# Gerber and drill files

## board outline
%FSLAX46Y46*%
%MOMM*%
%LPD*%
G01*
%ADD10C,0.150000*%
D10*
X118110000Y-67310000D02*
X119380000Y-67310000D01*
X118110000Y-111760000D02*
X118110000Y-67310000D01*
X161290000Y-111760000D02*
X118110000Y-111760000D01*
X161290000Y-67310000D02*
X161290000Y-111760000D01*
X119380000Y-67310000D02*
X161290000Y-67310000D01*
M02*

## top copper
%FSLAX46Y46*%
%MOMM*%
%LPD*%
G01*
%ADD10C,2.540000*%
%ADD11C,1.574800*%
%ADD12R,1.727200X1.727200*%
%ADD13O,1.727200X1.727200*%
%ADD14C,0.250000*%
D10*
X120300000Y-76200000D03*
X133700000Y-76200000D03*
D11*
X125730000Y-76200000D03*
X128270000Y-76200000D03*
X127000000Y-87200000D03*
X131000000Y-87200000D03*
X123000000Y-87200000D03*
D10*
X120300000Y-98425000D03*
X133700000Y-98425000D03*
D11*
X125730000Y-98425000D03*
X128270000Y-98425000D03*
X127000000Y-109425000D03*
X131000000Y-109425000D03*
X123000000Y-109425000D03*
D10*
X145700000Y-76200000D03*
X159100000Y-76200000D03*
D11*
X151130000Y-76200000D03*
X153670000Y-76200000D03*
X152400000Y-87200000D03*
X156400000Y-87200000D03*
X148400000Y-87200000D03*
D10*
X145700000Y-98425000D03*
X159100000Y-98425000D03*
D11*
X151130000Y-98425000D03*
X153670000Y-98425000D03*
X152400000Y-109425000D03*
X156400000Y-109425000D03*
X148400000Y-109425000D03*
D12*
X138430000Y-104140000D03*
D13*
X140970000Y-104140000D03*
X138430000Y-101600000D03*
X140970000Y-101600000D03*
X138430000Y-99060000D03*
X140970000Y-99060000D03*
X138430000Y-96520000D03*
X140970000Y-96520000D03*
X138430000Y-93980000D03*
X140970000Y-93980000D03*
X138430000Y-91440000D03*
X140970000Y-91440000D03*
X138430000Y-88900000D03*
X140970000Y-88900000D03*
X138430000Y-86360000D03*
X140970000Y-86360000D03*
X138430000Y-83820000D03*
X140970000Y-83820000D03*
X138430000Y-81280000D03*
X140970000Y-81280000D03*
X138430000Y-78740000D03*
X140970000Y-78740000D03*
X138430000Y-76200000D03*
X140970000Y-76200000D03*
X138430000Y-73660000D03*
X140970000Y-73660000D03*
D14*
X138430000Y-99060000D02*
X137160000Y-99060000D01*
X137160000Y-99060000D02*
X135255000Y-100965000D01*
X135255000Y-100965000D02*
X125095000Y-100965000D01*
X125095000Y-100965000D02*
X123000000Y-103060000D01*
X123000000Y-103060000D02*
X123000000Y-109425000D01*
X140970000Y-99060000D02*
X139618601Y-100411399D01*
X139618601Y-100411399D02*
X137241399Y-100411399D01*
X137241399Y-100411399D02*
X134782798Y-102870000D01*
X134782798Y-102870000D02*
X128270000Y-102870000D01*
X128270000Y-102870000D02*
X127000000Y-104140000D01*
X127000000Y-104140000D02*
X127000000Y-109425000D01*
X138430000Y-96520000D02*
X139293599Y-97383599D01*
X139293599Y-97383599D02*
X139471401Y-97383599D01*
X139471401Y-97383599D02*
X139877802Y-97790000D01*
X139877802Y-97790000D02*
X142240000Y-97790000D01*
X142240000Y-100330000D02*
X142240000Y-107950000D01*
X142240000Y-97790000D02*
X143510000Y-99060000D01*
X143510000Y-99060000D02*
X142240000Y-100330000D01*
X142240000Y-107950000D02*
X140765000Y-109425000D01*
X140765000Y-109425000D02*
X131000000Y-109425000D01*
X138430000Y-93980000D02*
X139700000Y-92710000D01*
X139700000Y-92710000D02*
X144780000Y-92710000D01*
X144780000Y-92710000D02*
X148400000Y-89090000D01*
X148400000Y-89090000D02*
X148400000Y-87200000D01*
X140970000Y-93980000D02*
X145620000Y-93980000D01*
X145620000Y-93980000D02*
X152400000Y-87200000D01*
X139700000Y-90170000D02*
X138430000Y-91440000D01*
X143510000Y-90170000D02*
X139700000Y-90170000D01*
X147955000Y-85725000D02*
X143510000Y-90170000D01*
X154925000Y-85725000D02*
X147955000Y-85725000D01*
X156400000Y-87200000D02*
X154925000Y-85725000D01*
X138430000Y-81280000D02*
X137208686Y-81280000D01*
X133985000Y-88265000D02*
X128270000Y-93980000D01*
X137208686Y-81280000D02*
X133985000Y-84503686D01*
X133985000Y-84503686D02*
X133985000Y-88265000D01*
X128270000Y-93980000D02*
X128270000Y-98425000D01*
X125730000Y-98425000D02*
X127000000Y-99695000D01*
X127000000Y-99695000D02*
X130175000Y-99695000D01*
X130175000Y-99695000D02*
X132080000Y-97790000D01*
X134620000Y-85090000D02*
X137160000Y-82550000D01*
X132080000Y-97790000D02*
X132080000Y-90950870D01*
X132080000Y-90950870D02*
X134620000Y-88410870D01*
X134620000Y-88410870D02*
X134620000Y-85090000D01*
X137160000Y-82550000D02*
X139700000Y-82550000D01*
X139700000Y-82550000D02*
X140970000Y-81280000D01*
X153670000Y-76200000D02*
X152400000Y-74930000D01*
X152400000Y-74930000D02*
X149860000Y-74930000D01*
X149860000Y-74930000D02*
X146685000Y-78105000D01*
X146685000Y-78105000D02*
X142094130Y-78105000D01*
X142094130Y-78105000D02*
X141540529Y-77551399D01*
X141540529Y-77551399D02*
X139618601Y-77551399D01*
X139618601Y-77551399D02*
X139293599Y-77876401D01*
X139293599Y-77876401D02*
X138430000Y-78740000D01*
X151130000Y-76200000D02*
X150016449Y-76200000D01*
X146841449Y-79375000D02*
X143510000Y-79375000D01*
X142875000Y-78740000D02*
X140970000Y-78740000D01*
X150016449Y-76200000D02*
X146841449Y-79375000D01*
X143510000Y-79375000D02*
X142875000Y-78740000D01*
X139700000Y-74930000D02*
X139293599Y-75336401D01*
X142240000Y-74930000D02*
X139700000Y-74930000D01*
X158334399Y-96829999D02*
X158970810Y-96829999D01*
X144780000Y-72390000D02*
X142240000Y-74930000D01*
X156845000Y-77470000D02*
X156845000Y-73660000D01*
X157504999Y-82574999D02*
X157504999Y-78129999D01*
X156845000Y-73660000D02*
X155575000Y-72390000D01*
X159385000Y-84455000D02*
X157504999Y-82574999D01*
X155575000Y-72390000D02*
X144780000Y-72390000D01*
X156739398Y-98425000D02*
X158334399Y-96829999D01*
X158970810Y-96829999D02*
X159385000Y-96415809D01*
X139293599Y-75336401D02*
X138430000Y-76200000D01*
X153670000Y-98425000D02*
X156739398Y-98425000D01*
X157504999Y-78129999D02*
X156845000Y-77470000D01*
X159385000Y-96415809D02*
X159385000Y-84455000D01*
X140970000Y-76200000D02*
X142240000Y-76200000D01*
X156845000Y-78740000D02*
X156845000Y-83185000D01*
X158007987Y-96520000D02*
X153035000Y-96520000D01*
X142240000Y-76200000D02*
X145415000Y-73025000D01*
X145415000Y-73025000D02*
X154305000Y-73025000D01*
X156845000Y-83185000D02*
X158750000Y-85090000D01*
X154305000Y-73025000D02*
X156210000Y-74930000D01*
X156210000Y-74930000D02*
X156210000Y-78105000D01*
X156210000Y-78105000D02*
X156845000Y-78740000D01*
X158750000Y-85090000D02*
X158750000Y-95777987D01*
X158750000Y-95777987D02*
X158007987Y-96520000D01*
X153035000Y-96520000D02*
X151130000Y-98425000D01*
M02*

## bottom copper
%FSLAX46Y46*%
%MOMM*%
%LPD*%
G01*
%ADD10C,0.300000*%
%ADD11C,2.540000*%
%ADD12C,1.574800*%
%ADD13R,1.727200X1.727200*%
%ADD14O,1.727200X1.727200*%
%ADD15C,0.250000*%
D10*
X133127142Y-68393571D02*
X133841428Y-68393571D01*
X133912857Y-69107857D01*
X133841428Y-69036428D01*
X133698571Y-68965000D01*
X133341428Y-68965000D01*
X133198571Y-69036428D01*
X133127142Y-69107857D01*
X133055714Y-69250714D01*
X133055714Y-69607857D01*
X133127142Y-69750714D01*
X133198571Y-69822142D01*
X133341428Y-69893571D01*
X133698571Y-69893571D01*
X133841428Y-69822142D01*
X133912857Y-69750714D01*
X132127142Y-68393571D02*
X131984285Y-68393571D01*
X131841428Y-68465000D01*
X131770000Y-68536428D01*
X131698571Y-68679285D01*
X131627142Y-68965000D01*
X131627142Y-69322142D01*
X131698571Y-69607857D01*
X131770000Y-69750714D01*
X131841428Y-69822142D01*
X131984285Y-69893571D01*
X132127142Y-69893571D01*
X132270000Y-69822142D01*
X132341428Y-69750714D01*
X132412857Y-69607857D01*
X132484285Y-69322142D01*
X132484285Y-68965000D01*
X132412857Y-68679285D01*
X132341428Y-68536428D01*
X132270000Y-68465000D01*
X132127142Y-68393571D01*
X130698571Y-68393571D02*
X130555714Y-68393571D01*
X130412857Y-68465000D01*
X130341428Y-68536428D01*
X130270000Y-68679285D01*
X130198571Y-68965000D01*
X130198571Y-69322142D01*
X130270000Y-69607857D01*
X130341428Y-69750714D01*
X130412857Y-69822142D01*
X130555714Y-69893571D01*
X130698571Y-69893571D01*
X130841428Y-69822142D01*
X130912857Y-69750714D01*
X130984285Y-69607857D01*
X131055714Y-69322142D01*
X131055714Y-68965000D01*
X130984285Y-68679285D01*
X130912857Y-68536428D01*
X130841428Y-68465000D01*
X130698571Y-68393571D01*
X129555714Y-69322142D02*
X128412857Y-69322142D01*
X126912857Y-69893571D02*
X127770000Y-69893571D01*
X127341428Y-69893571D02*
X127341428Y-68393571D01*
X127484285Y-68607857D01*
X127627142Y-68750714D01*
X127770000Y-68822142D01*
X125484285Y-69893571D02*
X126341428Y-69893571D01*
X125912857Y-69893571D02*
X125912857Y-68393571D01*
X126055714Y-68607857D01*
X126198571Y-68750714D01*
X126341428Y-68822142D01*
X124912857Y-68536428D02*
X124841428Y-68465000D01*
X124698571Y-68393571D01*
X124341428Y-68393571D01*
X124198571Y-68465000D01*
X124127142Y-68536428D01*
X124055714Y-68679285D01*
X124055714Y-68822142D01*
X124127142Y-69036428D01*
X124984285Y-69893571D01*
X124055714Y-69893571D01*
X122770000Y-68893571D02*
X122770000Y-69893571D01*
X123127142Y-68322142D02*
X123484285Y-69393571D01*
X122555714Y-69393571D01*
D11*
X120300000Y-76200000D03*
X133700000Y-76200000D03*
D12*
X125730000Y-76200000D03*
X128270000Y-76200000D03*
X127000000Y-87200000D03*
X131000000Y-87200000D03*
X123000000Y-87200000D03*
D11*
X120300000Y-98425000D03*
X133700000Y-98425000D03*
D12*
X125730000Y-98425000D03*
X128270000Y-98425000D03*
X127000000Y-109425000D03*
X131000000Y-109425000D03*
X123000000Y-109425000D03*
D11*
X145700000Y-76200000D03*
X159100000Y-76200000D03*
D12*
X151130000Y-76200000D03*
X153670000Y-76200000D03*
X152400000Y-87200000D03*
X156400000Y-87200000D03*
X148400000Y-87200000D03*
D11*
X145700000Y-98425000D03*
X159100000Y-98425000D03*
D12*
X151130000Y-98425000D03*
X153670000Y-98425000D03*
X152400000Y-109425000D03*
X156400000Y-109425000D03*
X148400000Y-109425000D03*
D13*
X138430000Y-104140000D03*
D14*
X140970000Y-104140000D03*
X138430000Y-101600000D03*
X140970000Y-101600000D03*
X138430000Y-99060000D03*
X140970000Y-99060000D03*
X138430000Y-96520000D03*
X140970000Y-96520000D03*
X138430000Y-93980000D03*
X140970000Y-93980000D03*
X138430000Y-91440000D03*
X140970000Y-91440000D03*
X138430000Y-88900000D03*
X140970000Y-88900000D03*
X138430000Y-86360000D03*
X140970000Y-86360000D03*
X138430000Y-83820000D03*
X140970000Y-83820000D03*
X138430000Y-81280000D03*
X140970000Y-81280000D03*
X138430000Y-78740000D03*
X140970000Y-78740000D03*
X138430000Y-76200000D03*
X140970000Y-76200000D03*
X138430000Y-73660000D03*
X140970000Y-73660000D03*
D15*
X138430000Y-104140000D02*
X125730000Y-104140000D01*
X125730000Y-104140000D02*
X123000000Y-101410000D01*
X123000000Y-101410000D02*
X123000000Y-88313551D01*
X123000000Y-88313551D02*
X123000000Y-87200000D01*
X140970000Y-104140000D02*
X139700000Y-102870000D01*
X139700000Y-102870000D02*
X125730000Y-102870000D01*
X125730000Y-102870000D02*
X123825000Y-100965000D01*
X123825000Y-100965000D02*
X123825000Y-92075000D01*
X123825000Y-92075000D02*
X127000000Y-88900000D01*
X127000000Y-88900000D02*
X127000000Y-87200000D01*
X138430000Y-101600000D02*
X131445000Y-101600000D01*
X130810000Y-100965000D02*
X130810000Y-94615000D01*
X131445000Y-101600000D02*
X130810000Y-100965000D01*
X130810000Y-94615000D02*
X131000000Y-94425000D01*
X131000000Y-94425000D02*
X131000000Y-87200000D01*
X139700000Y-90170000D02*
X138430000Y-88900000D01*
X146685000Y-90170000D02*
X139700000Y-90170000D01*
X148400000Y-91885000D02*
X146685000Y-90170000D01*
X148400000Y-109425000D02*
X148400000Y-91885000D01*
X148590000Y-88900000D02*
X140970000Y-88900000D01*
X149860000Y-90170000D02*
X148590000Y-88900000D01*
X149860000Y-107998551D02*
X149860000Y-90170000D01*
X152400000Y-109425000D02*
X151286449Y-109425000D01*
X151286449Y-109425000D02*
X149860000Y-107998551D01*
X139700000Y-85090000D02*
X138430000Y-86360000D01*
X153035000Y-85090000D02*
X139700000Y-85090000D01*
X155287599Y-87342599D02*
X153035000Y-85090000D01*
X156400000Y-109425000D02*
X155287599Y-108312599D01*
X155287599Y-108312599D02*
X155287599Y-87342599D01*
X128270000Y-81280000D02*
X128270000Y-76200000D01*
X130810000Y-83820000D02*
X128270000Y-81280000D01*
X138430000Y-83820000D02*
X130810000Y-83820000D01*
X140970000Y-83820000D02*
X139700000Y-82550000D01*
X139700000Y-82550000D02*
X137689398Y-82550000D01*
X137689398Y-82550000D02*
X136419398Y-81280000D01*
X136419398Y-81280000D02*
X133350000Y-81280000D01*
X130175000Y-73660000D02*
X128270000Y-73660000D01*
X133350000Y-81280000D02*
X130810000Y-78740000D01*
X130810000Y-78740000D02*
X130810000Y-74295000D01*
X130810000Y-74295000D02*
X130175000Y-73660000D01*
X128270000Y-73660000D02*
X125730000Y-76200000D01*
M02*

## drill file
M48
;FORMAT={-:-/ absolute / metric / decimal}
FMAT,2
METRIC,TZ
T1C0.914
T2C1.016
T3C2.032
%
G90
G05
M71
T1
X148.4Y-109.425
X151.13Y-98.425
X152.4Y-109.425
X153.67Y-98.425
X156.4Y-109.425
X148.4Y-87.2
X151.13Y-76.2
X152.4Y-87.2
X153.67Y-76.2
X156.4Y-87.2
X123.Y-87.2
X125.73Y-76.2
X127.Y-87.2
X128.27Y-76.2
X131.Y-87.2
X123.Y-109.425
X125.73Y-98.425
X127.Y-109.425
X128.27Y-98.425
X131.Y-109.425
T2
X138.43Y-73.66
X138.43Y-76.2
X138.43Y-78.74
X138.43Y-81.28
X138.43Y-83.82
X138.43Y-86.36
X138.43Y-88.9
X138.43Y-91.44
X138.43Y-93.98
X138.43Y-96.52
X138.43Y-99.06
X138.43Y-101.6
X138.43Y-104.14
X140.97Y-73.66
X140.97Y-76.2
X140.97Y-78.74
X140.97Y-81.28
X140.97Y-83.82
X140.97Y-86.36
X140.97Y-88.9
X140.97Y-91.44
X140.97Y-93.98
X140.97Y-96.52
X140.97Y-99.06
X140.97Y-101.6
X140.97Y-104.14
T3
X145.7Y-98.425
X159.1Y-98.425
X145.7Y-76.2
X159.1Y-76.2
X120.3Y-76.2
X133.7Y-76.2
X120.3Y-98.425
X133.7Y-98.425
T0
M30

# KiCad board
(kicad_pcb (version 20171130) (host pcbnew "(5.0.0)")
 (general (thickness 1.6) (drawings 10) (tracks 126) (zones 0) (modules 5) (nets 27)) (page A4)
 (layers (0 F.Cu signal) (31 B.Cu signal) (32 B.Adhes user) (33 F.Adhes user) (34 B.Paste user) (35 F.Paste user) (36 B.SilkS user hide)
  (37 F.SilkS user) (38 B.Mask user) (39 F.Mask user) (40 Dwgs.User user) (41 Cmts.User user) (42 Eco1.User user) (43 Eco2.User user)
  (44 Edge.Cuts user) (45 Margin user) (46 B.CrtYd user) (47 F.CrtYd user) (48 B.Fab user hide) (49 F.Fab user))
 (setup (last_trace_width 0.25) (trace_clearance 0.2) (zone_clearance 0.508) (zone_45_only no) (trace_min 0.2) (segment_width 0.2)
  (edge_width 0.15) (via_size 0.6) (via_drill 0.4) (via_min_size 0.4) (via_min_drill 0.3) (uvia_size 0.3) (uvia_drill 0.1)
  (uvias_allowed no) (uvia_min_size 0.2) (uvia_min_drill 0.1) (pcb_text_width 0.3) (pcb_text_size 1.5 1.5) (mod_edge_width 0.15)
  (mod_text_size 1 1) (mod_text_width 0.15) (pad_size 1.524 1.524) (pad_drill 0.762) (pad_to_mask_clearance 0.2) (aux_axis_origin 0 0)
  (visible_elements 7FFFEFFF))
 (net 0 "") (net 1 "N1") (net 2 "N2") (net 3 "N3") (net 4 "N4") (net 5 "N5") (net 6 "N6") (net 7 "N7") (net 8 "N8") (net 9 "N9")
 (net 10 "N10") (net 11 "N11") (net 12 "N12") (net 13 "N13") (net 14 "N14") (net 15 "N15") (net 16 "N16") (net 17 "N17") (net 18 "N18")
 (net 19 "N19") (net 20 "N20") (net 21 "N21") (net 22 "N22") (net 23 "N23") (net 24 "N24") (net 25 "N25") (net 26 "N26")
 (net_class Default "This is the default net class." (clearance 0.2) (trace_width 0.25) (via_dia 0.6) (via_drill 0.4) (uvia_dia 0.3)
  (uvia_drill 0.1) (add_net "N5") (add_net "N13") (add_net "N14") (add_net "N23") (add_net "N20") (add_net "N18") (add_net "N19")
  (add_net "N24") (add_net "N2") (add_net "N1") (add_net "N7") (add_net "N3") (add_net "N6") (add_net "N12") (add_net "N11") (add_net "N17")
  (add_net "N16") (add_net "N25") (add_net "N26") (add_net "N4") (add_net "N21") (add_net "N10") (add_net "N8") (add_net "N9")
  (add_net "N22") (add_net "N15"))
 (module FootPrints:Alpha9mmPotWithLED (layer F.Cu) (at 127 76.2)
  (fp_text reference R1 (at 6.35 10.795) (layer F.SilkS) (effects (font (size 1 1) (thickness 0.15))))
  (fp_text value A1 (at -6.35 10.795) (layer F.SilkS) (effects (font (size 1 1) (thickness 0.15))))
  (pad "" thru_hole circle (at -6.7 0) (size 2.54 2.54) (drill 2.032) (layers *.Cu *.Mask F.SilkS))
  (pad "" thru_hole circle (at 6.7 0) (size 2.54 2.54) (drill 2.032) (layers *.Cu *.Mask F.SilkS))
  (pad 4 thru_hole circle (at -1.27 0) (size 1.5748 1.5748) (drill 0.9144) (layers *.Cu *.Mask F.SilkS) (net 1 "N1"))
  (pad 5 thru_hole circle (at 1.27 0) (size 1.5748 1.5748) (drill 0.9144) (layers *.Cu *.Mask F.SilkS) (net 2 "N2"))
  (pad 2 thru_hole circle (at 0 11) (size 1.5748 1.5748) (drill 0.9144) (layers *.Cu *.Mask F.SilkS) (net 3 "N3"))
  (pad 3 thru_hole circle (at 4 11) (size 1.5748 1.5748) (drill 0.9144) (layers *.Cu *.Mask F.SilkS) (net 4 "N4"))
  (pad 1 thru_hole circle (at -4 11) (size 1.5748 1.5748) (drill 0.9144) (layers *.Cu *.Mask F.SilkS) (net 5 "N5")))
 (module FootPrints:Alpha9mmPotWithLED (layer F.Cu) (at 127 98.425)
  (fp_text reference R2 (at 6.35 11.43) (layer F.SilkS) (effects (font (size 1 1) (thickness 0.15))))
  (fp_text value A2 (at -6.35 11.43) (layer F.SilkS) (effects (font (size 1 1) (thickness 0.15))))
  (pad "" thru_hole circle (at -6.7 0) (size 2.54 2.54) (drill 2.032) (layers *.Cu *.Mask F.SilkS))
  (pad "" thru_hole circle (at 6.7 0) (size 2.54 2.54) (drill 2.032) (layers *.Cu *.Mask F.SilkS))
  (pad 4 thru_hole circle (at -1.27 0) (size 1.5748 1.5748) (drill 0.9144) (layers *.Cu *.Mask F.SilkS) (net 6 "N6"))
  (pad 5 thru_hole circle (at 1.27 0) (size 1.5748 1.5748) (drill 0.9144) (layers *.Cu *.Mask F.SilkS) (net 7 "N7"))
  (pad 2 thru_hole circle (at 0 11) (size 1.5748 1.5748) (drill 0.9144) (layers *.Cu *.Mask F.SilkS) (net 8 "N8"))
  (pad 3 thru_hole circle (at 4 11) (size 1.5748 1.5748) (drill 0.9144) (layers *.Cu *.Mask F.SilkS) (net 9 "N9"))
  (pad 1 thru_hole circle (at -4 11) (size 1.5748 1.5748) (drill 0.9144) (layers *.Cu *.Mask F.SilkS) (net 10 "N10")))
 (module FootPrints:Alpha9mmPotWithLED (layer F.Cu) (at 152.4 76.2)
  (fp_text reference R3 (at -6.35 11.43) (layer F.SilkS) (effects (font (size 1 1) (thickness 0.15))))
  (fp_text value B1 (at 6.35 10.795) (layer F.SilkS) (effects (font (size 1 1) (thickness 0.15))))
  (pad "" thru_hole circle (at -6.7 0) (size 2.54 2.54) (drill 2.032) (layers *.Cu *.Mask F.SilkS))
  (pad "" thru_hole circle (at 6.7 0) (size 2.54 2.54) (drill 2.032) (layers *.Cu *.Mask F.SilkS))
  (pad 4 thru_hole circle (at -1.27 0) (size 1.5748 1.5748) (drill 0.9144) (layers *.Cu *.Mask F.SilkS) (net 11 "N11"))
  (pad 5 thru_hole circle (at 1.27 0) (size 1.5748 1.5748) (drill 0.9144) (layers *.Cu *.Mask F.SilkS) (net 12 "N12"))
  (pad 2 thru_hole circle (at 0 11) (size 1.5748 1.5748) (drill 0.9144) (layers *.Cu *.Mask F.SilkS) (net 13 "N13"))
  (pad 3 thru_hole circle (at 4 11) (size 1.5748 1.5748) (drill 0.9144) (layers *.Cu *.Mask F.SilkS) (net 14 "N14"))
  (pad 1 thru_hole circle (at -4 11) (size 1.5748 1.5748) (drill 0.9144) (layers *.Cu *.Mask F.SilkS) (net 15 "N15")))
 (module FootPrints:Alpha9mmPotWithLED (layer F.Cu) (at 152.4 98.425)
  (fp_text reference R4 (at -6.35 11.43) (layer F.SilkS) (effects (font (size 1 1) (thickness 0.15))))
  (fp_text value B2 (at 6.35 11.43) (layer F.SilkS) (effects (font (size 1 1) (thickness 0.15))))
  (pad "" thru_hole circle (at -6.7 0) (size 2.54 2.54) (drill 2.032) (layers *.Cu *.Mask F.SilkS))
  (pad "" thru_hole circle (at 6.7 0) (size 2.54 2.54) (drill 2.032) (layers *.Cu *.Mask F.SilkS))
  (pad 4 thru_hole circle (at -1.27 0) (size 1.5748 1.5748) (drill 0.9144) (layers *.Cu *.Mask F.SilkS) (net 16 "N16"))
  (pad 5 thru_hole circle (at 1.27 0) (size 1.5748 1.5748) (drill 0.9144) (layers *.Cu *.Mask F.SilkS) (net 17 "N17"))
  (pad 2 thru_hole circle (at 0 11) (size 1.5748 1.5748) (drill 0.9144) (layers *.Cu *.Mask F.SilkS) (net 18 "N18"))
  (pad 3 thru_hole circle (at 4 11) (size 1.5748 1.5748) (drill 0.9144) (layers *.Cu *.Mask F.SilkS) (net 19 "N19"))
  (pad 1 thru_hole circle (at -4 11) (size 1.5748 1.5748) (drill 0.9144) (layers *.Cu *.Mask F.SilkS) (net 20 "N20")))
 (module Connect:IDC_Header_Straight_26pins (layer B.Cu) (at 138.43 104.14 90)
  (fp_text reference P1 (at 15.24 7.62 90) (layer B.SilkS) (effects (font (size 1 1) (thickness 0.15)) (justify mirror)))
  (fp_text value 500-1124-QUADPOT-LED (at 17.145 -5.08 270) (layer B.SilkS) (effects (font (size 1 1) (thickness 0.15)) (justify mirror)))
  (pad 1 thru_hole rect (at 0 0 90) (size 1.7272 1.7272) (drill 1.016) (layers *.Cu *.Mask) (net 5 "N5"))
  (pad 2 thru_hole oval (at 0 2.54 90) (size 1.7272 1.7272) (drill 1.016) (layers *.Cu *.Mask) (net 3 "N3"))
  (pad 3 thru_hole oval (at 2.54 0 90) (size 1.7272 1.7272) (drill 1.016) (layers *.Cu *.Mask) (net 4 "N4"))
  (pad 4 thru_hole oval (at 2.54 2.54 90) (size 1.7272 1.7272) (drill 1.016) (layers *.Cu *.Mask) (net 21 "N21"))
  (pad 5 thru_hole oval (at 5.08 0 90) (size 1.7272 1.7272) (drill 1.016) (layers *.Cu *.Mask) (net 10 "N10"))
  (pad 6 thru_hole oval (at 5.08 2.54 90) (size 1.7272 1.7272) (drill 1.016) (layers *.Cu *.Mask) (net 8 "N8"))
  (pad 7 thru_hole oval (at 7.62 0 90) (size 1.7272 1.7272) (drill 1.016) (layers *.Cu *.Mask) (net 9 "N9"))
  (pad 8 thru_hole oval (at 7.62 2.54 90) (size 1.7272 1.7272) (drill 1.016) (layers *.Cu *.Mask) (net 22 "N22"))
  (pad 9 thru_hole oval (at 10.16 0 90) (size 1.7272 1.7272) (drill 1.016) (layers *.Cu *.Mask) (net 15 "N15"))
  (pad 10 thru_hole oval (at 10.16 2.54 90) (size 1.7272 1.7272) (drill 1.016) (layers *.Cu *.Mask) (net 13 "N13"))
  (pad 11 thru_hole oval (at 12.7 0 90) (size 1.7272 1.7272) (drill 1.016) (layers *.Cu *.Mask) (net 14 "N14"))
  (pad 12 thru_hole oval (at 12.7 2.54 90) (size 1.7272 1.7272) (drill 1.016) (layers *.Cu *.Mask) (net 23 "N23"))
  (pad 13 thru_hole oval (at 15.24 0 90) (size 1.7272 1.7272) (drill 1.016) (layers *.Cu *.Mask) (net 20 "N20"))
  (pad 14 thru_hole oval (at 15.24 2.54 90) (size 1.7272 1.7272) (drill 1.016) (layers *.Cu *.Mask) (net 18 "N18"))
  (pad 15 thru_hole oval (at 17.78 0 90) (size 1.7272 1.7272) (drill 1.016) (layers *.Cu *.Mask) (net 19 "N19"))
  (pad 16 thru_hole oval (at 17.78 2.54 90) (size 1.7272 1.7272) (drill 1.016) (layers *.Cu *.Mask) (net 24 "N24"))
  (pad 17 thru_hole oval (at 20.32 0 90) (size 1.7272 1.7272) (drill 1.016) (layers *.Cu *.Mask) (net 2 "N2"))
  (pad 18 thru_hole oval (at 20.32 2.54 90) (size 1.7272 1.7272) (drill 1.016) (layers *.Cu *.Mask) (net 1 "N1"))
  (pad 19 thru_hole oval (at 22.86 0 90) (size 1.7272 1.7272) (drill 1.016) (layers *.Cu *.Mask) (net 7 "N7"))
  (pad 20 thru_hole oval (at 22.86 2.54 90) (size 1.7272 1.7272) (drill 1.016) (layers *.Cu *.Mask) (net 6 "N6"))
  (pad 21 thru_hole oval (at 25.4 0 90) (size 1.7272 1.7272) (drill 1.016) (layers *.Cu *.Mask) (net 12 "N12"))
  (pad 22 thru_hole oval (at 25.4 2.54 90) (size 1.7272 1.7272) (drill 1.016) (layers *.Cu *.Mask) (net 11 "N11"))
  (pad 23 thru_hole oval (at 27.94 0 90) (size 1.7272 1.7272) (drill 1.016) (layers *.Cu *.Mask) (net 17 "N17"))
  (pad 24 thru_hole oval (at 27.94 2.54 90) (size 1.7272 1.7272) (drill 1.016) (layers *.Cu *.Mask) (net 16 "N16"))
  (pad 25 thru_hole oval (at 30.48 0 90) (size 1.7272 1.7272) (drill 1.016) (layers *.Cu *.Mask) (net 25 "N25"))
  (pad 26 thru_hole oval (at 30.48 2.54 90) (size 1.7272 1.7272) (drill 1.016) (layers *.Cu *.Mask) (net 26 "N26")))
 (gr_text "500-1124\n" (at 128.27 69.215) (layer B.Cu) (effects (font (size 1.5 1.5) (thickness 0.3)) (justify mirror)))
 (gr_line (start 118.11 67.31) (end 119.38 67.31) (angle 90) (layer Edge.Cuts) (width 0.15))
 (gr_line (start 118.11 111.76) (end 118.11 67.31) (angle 90) (layer Edge.Cuts) (width 0.15))
 (gr_line (start 161.29 111.76) (end 118.11 111.76) (angle 90) (layer Edge.Cuts) (width 0.15))
 (gr_line (start 161.29 67.31) (end 161.29 111.76) (angle 90) (layer Edge.Cuts) (width 0.15))
 (gr_line (start 119.38 67.31) (end 161.29 67.31) (angle 90) (layer Edge.Cuts) (width 0.15))
 (segment (start 138.43 104.14) (end 125.73 104.14) (width 0.25) (layer B.Cu) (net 5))
 (segment (start 125.73 104.14) (end 123 101.41) (width 0.25) (layer B.Cu) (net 5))
 (segment (start 123 101.41) (end 123 88.313551) (width 0.25) (layer B.Cu) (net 5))
 (segment (start 123 88.313551) (end 123 87.2) (width 0.25) (layer B.Cu) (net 5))
 (segment (start 140.97 104.14) (end 139.7 102.87) (width 0.25) (layer B.Cu) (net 3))
 (segment (start 139.7 102.87) (end 125.73 102.87) (width 0.25) (layer B.Cu) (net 3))
 (segment (start 125.73 102.87) (end 123.825 100.965) (width 0.25) (layer B.Cu) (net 3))
 (segment (start 123.825 100.965) (end 123.825 92.075) (width 0.25) (layer B.Cu) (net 3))
 (segment (start 123.825 92.075) (end 127 88.9) (width 0.25) (layer B.Cu) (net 3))
 (segment (start 127 88.9) (end 127 87.2) (width 0.25) (layer B.Cu) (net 3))
 (segment (start 138.43 101.6) (end 131.445 101.6) (width 0.25) (layer B.Cu) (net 4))
 (segment (start 130.81 100.965) (end 130.81 94.615) (width 0.25) (layer B.Cu) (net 4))
 (segment (start 131.445 101.6) (end 130.81 100.965) (width 0.25) (layer B.Cu) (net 4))
 (segment (start 130.81 94.615) (end 131 94.425) (width 0.25) (layer B.Cu) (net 4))
 (segment (start 131 94.425) (end 131 87.2) (width 0.25) (layer B.Cu) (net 4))
 (segment (start 138.43 99.06) (end 137.16 99.06) (width 0.25) (layer F.Cu) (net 10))
 (segment (start 137.16 99.06) (end 135.255 100.965) (width 0.25) (layer F.Cu) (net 10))
 (segment (start 135.255 100.965) (end 125.095 100.965) (width 0.25) (layer F.Cu) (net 10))
 (segment (start 125.095 100.965) (end 123 103.06) (width 0.25) (layer F.Cu) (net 10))
 (segment (start 123 103.06) (end 123 109.425) (width 0.25) (layer F.Cu) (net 10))
 (segment (start 140.97 99.06) (end 139.618601 100.411399) (width 0.25) (layer F.Cu) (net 8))
 (segment (start 139.618601 100.411399) (end 137.241399 100.411399) (width 0.25) (layer F.Cu) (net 8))
 (segment (start 137.241399 100.411399) (end 134.782798 102.87) (width 0.25) (layer F.Cu) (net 8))
 (segment (start 134.782798 102.87) (end 128.27 102.87) (width 0.25) (layer F.Cu) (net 8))
 (segment (start 128.27 102.87) (end 127 104.14) (width 0.25) (layer F.Cu) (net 8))
 (segment (start 127 104.14) (end 127 109.425) (width 0.25) (layer F.Cu) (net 8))
 (segment (start 138.43 96.52) (end 139.293599 97.383599) (width 0.25) (layer F.Cu) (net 9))
 (segment (start 139.293599 97.383599) (end 139.471401 97.383599) (width 0.25) (layer F.Cu) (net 9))
 (segment (start 139.471401 97.383599) (end 139.877802 97.79) (width 0.25) (layer F.Cu) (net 9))
 (segment (start 139.877802 97.79) (end 142.24 97.79) (width 0.25) (layer F.Cu) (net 9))
 (segment (start 142.24 100.33) (end 142.24 107.95) (width 0.25) (layer F.Cu) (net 9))
 (segment (start 142.24 97.79) (end 143.51 99.06) (width 0.25) (layer F.Cu) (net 9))
 (segment (start 143.51 99.06) (end 142.24 100.33) (width 0.25) (layer F.Cu) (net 9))
 (segment (start 142.24 107.95) (end 140.765 109.425) (width 0.25) (layer F.Cu) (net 9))
 (segment (start 140.765 109.425) (end 131 109.425) (width 0.25) (layer F.Cu) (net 9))
 (segment (start 138.43 93.98) (end 139.7 92.71) (width 0.25) (layer F.Cu) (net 15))
 (segment (start 139.7 92.71) (end 144.78 92.71) (width 0.25) (layer F.Cu) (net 15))
 (segment (start 144.78 92.71) (end 148.4 89.09) (width 0.25) (layer F.Cu) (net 15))
 (segment (start 148.4 89.09) (end 148.4 87.2) (width 0.25) (layer F.Cu) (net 15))
 (segment (start 140.97 93.98) (end 145.62 93.98) (width 0.25) (layer F.Cu) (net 13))
 (segment (start 145.62 93.98) (end 152.4 87.2) (width 0.25) (layer F.Cu) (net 13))
 (segment (start 139.7 90.17) (end 138.43 91.44) (width 0.25) (layer F.Cu) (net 14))
 (segment (start 143.51 90.17) (end 139.7 90.17) (width 0.25) (layer F.Cu) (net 14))
 (segment (start 147.955 85.725) (end 143.51 90.17) (width 0.25) (layer F.Cu) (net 14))
 (segment (start 154.925 85.725) (end 147.955 85.725) (width 0.25) (layer F.Cu) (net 14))
 (segment (start 156.4 87.2) (end 154.925 85.725) (width 0.25) (layer F.Cu) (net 14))
 (segment (start 139.7 90.17) (end 138.43 88.9) (width 0.25) (layer B.Cu) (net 20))
 (segment (start 146.685 90.17) (end 139.7 90.17) (width 0.25) (layer B.Cu) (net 20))
 (segment (start 148.4 91.885) (end 146.685 90.17) (width 0.25) (layer B.Cu) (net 20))
 (segment (start 148.4 109.425) (end 148.4 91.885) (width 0.25) (layer B.Cu) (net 20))
 (segment (start 148.59 88.9) (end 140.97 88.9) (width 0.25) (layer B.Cu) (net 18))
 (segment (start 149.86 90.17) (end 148.59 88.9) (width 0.25) (layer B.Cu) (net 18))
 (segment (start 149.86 107.998551) (end 149.86 90.17) (width 0.25) (layer B.Cu) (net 18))
 (segment (start 152.4 109.425) (end 151.286449 109.425) (width 0.25) (layer B.Cu) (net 18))
 (segment (start 151.286449 109.425) (end 149.86 107.998551) (width 0.25) (layer B.Cu) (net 18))
 (segment (start 139.7 85.09) (end 138.43 86.36) (width 0.25) (layer B.Cu) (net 19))
 (segment (start 153.035 85.09) (end 139.7 85.09) (width 0.25) (layer B.Cu) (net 19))
 (segment (start 155.287599 87.342599) (end 153.035 85.09) (width 0.25) (layer B.Cu) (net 19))
 (segment (start 156.4 109.425) (end 155.287599 108.312599) (width 0.25) (layer B.Cu) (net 19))
 (segment (start 155.287599 108.312599) (end 155.287599 87.342599) (width 0.25) (layer B.Cu) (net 19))
 (segment (start 128.27 81.28) (end 128.27 76.2) (width 0.25) (layer B.Cu) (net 2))
 (segment (start 130.81 83.82) (end 128.27 81.28) (width 0.25) (layer B.Cu) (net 2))
 (segment (start 138.43 83.82) (end 130.81 83.82) (width 0.25) (layer B.Cu) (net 2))
 (segment (start 140.97 83.82) (end 139.7 82.55) (width 0.25) (layer B.Cu) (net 1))
 (segment (start 139.7 82.55) (end 137.689398 82.55) (width 0.25) (layer B.Cu) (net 1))
 (segment (start 137.689398 82.55) (end 136.419398 81.28) (width 0.25) (layer B.Cu) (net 1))
 (segment (start 136.419398 81.28) (end 133.35 81.28) (width 0.25) (layer B.Cu) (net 1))
 (segment (start 130.175 73.66) (end 128.27 73.66) (width 0.25) (layer B.Cu) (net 1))
 (segment (start 133.35 81.28) (end 130.81 78.74) (width 0.25) (layer B.Cu) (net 1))
 (segment (start 130.81 78.74) (end 130.81 74.295) (width 0.25) (layer B.Cu) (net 1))
 (segment (start 130.81 74.295) (end 130.175 73.66) (width 0.25) (layer B.Cu) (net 1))
 (segment (start 128.27 73.66) (end 125.73 76.2) (width 0.25) (layer B.Cu) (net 1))
 (segment (start 138.43 81.28) (end 137.208686 81.28) (width 0.25) (layer F.Cu) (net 7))
 (segment (start 133.985 88.265) (end 128.27 93.98) (width 0.25) (layer F.Cu) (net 7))
 (segment (start 137.208686 81.28) (end 133.985 84.503686) (width 0.25) (layer F.Cu) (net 7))
 (segment (start 133.985 84.503686) (end 133.985 88.265) (width 0.25) (layer F.Cu) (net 7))
 (segment (start 128.27 93.98) (end 128.27 98.425) (width 0.25) (layer F.Cu) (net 7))
 (segment (start 125.73 98.425) (end 127 99.695) (width 0.25) (layer F.Cu) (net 6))
 (segment (start 127 99.695) (end 130.175 99.695) (width 0.25) (layer F.Cu) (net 6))
 (segment (start 130.175 99.695) (end 132.08 97.79) (width 0.25) (layer F.Cu) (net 6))
 (segment (start 134.62 85.09) (end 137.16 82.55) (width 0.25) (layer F.Cu) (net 6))
 (segment (start 132.08 97.79) (end 132.08 90.95087) (width 0.25) (layer F.Cu) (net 6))
 (segment (start 132.08 90.95087) (end 134.62 88.41087) (width 0.25) (layer F.Cu) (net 6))
 (segment (start 134.62 88.41087) (end 134.62 85.09) (width 0.25) (layer F.Cu) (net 6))
 (segment (start 137.16 82.55) (end 139.7 82.55) (width 0.25) (layer F.Cu) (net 6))
 (segment (start 139.7 82.55) (end 140.97 81.28) (width 0.25) (layer F.Cu) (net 6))
 (segment (start 153.67 76.2) (end 152.4 74.93) (width 0.25) (layer F.Cu) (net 12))
 (segment (start 152.4 74.93) (end 149.86 74.93) (width 0.25) (layer F.Cu) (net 12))
 (segment (start 149.86 74.93) (end 146.685 78.105) (width 0.25) (layer F.Cu) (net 12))
 (segment (start 146.685 78.105) (end 142.09413 78.105) (width 0.25) (layer F.Cu) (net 12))
 (segment (start 142.09413 78.105) (end 141.540529 77.551399) (width 0.25) (layer F.Cu) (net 12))
 (segment (start 141.540529 77.551399) (end 139.618601 77.551399) (width 0.25) (layer F.Cu) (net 12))
 (segment (start 139.618601 77.551399) (end 139.293599 77.876401) (width 0.25) (layer F.Cu) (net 12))
 (segment (start 139.293599 77.876401) (end 138.43 78.74) (width 0.25) (layer F.Cu) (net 12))
 (segment (start 151.13 76.2) (end 150.016449 76.2) (width 0.25) (layer F.Cu) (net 11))
 (segment (start 146.841449 79.375) (end 143.51 79.375) (width 0.25) (layer F.Cu) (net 11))
 (segment (start 142.875 78.74) (end 140.97 78.74) (width 0.25) (layer F.Cu) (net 11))
 (segment (start 150.016449 76.2) (end 146.841449 79.375) (width 0.25) (layer F.Cu) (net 11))
 (segment (start 143.51 79.375) (end 142.875 78.74) (width 0.25) (layer F.Cu) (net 11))
 (segment (start 139.7 74.93) (end 139.293599 75.336401) (width 0.25) (layer F.Cu) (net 17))
 (segment (start 142.24 74.93) (end 139.7 74.93) (width 0.25) (layer F.Cu) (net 17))
 (segment (start 158.334399 96.829999) (end 158.97081 96.829999) (width 0.25) (layer F.Cu) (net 17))
 (segment (start 144.78 72.39) (end 142.24 74.93) (width 0.25) (layer F.Cu) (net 17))
 (segment (start 156.845 77.47) (end 156.845 73.66) (width 0.25) (layer F.Cu) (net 17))
 (segment (start 157.504999 82.574999) (end 157.504999 78.129999) (width 0.25) (layer F.Cu) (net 17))
 (segment (start 156.845 73.66) (end 155.575 72.39) (width 0.25) (layer F.Cu) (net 17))
 (segment (start 159.385 84.455) (end 157.504999 82.574999) (width 0.25) (layer F.Cu) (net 17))
 (segment (start 155.575 72.39) (end 144.78 72.39) (width 0.25) (layer F.Cu) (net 17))
 (segment (start 156.739398 98.425) (end 158.334399 96.829999) (width 0.25) (layer F.Cu) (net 17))
 (segment (start 158.97081 96.829999) (end 159.385 96.415809) (width 0.25) (layer F.Cu) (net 17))
 (segment (start 139.293599 75.336401) (end 138.43 76.2) (width 0.25) (layer F.Cu) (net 17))
 (segment (start 153.67 98.425) (end 156.739398 98.425) (width 0.25) (layer F.Cu) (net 17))
 (segment (start 157.504999 78.129999) (end 156.845 77.47) (width 0.25) (layer F.Cu) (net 17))
 (segment (start 159.385 96.415809) (end 159.385 84.455) (width 0.25) (layer F.Cu) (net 17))
 (segment (start 140.97 76.2) (end 142.24 76.2) (width 0.25) (layer F.Cu) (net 16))
 (segment (start 156.845 78.74) (end 156.845 83.185) (width 0.25) (layer F.Cu) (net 16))
 (segment (start 158.007987 96.52) (end 153.035 96.52) (width 0.25) (layer F.Cu) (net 16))
 (segment (start 142.24 76.2) (end 145.415 73.025) (width 0.25) (layer F.Cu) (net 16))
 (segment (start 145.415 73.025) (end 154.305 73.025) (width 0.25) (layer F.Cu) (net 16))
 (segment (start 156.845 83.185) (end 158.75 85.09) (width 0.25) (layer F.Cu) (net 16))
 (segment (start 154.305 73.025) (end 156.21 74.93) (width 0.25) (layer F.Cu) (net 16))
 (segment (start 156.21 74.93) (end 156.21 78.105) (width 0.25) (layer F.Cu) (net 16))
 (segment (start 156.21 78.105) (end 156.845 78.74) (width 0.25) (layer F.Cu) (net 16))
 (segment (start 158.75 85.09) (end 158.75 95.777987) (width 0.25) (layer F.Cu) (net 16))
 (segment (start 158.75 95.777987) (end 158.007987 96.52) (width 0.25) (layer F.Cu) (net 16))
 (segment (start 153.035 96.52) (end 151.13 98.425) (width 0.25) (layer F.Cu) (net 16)))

